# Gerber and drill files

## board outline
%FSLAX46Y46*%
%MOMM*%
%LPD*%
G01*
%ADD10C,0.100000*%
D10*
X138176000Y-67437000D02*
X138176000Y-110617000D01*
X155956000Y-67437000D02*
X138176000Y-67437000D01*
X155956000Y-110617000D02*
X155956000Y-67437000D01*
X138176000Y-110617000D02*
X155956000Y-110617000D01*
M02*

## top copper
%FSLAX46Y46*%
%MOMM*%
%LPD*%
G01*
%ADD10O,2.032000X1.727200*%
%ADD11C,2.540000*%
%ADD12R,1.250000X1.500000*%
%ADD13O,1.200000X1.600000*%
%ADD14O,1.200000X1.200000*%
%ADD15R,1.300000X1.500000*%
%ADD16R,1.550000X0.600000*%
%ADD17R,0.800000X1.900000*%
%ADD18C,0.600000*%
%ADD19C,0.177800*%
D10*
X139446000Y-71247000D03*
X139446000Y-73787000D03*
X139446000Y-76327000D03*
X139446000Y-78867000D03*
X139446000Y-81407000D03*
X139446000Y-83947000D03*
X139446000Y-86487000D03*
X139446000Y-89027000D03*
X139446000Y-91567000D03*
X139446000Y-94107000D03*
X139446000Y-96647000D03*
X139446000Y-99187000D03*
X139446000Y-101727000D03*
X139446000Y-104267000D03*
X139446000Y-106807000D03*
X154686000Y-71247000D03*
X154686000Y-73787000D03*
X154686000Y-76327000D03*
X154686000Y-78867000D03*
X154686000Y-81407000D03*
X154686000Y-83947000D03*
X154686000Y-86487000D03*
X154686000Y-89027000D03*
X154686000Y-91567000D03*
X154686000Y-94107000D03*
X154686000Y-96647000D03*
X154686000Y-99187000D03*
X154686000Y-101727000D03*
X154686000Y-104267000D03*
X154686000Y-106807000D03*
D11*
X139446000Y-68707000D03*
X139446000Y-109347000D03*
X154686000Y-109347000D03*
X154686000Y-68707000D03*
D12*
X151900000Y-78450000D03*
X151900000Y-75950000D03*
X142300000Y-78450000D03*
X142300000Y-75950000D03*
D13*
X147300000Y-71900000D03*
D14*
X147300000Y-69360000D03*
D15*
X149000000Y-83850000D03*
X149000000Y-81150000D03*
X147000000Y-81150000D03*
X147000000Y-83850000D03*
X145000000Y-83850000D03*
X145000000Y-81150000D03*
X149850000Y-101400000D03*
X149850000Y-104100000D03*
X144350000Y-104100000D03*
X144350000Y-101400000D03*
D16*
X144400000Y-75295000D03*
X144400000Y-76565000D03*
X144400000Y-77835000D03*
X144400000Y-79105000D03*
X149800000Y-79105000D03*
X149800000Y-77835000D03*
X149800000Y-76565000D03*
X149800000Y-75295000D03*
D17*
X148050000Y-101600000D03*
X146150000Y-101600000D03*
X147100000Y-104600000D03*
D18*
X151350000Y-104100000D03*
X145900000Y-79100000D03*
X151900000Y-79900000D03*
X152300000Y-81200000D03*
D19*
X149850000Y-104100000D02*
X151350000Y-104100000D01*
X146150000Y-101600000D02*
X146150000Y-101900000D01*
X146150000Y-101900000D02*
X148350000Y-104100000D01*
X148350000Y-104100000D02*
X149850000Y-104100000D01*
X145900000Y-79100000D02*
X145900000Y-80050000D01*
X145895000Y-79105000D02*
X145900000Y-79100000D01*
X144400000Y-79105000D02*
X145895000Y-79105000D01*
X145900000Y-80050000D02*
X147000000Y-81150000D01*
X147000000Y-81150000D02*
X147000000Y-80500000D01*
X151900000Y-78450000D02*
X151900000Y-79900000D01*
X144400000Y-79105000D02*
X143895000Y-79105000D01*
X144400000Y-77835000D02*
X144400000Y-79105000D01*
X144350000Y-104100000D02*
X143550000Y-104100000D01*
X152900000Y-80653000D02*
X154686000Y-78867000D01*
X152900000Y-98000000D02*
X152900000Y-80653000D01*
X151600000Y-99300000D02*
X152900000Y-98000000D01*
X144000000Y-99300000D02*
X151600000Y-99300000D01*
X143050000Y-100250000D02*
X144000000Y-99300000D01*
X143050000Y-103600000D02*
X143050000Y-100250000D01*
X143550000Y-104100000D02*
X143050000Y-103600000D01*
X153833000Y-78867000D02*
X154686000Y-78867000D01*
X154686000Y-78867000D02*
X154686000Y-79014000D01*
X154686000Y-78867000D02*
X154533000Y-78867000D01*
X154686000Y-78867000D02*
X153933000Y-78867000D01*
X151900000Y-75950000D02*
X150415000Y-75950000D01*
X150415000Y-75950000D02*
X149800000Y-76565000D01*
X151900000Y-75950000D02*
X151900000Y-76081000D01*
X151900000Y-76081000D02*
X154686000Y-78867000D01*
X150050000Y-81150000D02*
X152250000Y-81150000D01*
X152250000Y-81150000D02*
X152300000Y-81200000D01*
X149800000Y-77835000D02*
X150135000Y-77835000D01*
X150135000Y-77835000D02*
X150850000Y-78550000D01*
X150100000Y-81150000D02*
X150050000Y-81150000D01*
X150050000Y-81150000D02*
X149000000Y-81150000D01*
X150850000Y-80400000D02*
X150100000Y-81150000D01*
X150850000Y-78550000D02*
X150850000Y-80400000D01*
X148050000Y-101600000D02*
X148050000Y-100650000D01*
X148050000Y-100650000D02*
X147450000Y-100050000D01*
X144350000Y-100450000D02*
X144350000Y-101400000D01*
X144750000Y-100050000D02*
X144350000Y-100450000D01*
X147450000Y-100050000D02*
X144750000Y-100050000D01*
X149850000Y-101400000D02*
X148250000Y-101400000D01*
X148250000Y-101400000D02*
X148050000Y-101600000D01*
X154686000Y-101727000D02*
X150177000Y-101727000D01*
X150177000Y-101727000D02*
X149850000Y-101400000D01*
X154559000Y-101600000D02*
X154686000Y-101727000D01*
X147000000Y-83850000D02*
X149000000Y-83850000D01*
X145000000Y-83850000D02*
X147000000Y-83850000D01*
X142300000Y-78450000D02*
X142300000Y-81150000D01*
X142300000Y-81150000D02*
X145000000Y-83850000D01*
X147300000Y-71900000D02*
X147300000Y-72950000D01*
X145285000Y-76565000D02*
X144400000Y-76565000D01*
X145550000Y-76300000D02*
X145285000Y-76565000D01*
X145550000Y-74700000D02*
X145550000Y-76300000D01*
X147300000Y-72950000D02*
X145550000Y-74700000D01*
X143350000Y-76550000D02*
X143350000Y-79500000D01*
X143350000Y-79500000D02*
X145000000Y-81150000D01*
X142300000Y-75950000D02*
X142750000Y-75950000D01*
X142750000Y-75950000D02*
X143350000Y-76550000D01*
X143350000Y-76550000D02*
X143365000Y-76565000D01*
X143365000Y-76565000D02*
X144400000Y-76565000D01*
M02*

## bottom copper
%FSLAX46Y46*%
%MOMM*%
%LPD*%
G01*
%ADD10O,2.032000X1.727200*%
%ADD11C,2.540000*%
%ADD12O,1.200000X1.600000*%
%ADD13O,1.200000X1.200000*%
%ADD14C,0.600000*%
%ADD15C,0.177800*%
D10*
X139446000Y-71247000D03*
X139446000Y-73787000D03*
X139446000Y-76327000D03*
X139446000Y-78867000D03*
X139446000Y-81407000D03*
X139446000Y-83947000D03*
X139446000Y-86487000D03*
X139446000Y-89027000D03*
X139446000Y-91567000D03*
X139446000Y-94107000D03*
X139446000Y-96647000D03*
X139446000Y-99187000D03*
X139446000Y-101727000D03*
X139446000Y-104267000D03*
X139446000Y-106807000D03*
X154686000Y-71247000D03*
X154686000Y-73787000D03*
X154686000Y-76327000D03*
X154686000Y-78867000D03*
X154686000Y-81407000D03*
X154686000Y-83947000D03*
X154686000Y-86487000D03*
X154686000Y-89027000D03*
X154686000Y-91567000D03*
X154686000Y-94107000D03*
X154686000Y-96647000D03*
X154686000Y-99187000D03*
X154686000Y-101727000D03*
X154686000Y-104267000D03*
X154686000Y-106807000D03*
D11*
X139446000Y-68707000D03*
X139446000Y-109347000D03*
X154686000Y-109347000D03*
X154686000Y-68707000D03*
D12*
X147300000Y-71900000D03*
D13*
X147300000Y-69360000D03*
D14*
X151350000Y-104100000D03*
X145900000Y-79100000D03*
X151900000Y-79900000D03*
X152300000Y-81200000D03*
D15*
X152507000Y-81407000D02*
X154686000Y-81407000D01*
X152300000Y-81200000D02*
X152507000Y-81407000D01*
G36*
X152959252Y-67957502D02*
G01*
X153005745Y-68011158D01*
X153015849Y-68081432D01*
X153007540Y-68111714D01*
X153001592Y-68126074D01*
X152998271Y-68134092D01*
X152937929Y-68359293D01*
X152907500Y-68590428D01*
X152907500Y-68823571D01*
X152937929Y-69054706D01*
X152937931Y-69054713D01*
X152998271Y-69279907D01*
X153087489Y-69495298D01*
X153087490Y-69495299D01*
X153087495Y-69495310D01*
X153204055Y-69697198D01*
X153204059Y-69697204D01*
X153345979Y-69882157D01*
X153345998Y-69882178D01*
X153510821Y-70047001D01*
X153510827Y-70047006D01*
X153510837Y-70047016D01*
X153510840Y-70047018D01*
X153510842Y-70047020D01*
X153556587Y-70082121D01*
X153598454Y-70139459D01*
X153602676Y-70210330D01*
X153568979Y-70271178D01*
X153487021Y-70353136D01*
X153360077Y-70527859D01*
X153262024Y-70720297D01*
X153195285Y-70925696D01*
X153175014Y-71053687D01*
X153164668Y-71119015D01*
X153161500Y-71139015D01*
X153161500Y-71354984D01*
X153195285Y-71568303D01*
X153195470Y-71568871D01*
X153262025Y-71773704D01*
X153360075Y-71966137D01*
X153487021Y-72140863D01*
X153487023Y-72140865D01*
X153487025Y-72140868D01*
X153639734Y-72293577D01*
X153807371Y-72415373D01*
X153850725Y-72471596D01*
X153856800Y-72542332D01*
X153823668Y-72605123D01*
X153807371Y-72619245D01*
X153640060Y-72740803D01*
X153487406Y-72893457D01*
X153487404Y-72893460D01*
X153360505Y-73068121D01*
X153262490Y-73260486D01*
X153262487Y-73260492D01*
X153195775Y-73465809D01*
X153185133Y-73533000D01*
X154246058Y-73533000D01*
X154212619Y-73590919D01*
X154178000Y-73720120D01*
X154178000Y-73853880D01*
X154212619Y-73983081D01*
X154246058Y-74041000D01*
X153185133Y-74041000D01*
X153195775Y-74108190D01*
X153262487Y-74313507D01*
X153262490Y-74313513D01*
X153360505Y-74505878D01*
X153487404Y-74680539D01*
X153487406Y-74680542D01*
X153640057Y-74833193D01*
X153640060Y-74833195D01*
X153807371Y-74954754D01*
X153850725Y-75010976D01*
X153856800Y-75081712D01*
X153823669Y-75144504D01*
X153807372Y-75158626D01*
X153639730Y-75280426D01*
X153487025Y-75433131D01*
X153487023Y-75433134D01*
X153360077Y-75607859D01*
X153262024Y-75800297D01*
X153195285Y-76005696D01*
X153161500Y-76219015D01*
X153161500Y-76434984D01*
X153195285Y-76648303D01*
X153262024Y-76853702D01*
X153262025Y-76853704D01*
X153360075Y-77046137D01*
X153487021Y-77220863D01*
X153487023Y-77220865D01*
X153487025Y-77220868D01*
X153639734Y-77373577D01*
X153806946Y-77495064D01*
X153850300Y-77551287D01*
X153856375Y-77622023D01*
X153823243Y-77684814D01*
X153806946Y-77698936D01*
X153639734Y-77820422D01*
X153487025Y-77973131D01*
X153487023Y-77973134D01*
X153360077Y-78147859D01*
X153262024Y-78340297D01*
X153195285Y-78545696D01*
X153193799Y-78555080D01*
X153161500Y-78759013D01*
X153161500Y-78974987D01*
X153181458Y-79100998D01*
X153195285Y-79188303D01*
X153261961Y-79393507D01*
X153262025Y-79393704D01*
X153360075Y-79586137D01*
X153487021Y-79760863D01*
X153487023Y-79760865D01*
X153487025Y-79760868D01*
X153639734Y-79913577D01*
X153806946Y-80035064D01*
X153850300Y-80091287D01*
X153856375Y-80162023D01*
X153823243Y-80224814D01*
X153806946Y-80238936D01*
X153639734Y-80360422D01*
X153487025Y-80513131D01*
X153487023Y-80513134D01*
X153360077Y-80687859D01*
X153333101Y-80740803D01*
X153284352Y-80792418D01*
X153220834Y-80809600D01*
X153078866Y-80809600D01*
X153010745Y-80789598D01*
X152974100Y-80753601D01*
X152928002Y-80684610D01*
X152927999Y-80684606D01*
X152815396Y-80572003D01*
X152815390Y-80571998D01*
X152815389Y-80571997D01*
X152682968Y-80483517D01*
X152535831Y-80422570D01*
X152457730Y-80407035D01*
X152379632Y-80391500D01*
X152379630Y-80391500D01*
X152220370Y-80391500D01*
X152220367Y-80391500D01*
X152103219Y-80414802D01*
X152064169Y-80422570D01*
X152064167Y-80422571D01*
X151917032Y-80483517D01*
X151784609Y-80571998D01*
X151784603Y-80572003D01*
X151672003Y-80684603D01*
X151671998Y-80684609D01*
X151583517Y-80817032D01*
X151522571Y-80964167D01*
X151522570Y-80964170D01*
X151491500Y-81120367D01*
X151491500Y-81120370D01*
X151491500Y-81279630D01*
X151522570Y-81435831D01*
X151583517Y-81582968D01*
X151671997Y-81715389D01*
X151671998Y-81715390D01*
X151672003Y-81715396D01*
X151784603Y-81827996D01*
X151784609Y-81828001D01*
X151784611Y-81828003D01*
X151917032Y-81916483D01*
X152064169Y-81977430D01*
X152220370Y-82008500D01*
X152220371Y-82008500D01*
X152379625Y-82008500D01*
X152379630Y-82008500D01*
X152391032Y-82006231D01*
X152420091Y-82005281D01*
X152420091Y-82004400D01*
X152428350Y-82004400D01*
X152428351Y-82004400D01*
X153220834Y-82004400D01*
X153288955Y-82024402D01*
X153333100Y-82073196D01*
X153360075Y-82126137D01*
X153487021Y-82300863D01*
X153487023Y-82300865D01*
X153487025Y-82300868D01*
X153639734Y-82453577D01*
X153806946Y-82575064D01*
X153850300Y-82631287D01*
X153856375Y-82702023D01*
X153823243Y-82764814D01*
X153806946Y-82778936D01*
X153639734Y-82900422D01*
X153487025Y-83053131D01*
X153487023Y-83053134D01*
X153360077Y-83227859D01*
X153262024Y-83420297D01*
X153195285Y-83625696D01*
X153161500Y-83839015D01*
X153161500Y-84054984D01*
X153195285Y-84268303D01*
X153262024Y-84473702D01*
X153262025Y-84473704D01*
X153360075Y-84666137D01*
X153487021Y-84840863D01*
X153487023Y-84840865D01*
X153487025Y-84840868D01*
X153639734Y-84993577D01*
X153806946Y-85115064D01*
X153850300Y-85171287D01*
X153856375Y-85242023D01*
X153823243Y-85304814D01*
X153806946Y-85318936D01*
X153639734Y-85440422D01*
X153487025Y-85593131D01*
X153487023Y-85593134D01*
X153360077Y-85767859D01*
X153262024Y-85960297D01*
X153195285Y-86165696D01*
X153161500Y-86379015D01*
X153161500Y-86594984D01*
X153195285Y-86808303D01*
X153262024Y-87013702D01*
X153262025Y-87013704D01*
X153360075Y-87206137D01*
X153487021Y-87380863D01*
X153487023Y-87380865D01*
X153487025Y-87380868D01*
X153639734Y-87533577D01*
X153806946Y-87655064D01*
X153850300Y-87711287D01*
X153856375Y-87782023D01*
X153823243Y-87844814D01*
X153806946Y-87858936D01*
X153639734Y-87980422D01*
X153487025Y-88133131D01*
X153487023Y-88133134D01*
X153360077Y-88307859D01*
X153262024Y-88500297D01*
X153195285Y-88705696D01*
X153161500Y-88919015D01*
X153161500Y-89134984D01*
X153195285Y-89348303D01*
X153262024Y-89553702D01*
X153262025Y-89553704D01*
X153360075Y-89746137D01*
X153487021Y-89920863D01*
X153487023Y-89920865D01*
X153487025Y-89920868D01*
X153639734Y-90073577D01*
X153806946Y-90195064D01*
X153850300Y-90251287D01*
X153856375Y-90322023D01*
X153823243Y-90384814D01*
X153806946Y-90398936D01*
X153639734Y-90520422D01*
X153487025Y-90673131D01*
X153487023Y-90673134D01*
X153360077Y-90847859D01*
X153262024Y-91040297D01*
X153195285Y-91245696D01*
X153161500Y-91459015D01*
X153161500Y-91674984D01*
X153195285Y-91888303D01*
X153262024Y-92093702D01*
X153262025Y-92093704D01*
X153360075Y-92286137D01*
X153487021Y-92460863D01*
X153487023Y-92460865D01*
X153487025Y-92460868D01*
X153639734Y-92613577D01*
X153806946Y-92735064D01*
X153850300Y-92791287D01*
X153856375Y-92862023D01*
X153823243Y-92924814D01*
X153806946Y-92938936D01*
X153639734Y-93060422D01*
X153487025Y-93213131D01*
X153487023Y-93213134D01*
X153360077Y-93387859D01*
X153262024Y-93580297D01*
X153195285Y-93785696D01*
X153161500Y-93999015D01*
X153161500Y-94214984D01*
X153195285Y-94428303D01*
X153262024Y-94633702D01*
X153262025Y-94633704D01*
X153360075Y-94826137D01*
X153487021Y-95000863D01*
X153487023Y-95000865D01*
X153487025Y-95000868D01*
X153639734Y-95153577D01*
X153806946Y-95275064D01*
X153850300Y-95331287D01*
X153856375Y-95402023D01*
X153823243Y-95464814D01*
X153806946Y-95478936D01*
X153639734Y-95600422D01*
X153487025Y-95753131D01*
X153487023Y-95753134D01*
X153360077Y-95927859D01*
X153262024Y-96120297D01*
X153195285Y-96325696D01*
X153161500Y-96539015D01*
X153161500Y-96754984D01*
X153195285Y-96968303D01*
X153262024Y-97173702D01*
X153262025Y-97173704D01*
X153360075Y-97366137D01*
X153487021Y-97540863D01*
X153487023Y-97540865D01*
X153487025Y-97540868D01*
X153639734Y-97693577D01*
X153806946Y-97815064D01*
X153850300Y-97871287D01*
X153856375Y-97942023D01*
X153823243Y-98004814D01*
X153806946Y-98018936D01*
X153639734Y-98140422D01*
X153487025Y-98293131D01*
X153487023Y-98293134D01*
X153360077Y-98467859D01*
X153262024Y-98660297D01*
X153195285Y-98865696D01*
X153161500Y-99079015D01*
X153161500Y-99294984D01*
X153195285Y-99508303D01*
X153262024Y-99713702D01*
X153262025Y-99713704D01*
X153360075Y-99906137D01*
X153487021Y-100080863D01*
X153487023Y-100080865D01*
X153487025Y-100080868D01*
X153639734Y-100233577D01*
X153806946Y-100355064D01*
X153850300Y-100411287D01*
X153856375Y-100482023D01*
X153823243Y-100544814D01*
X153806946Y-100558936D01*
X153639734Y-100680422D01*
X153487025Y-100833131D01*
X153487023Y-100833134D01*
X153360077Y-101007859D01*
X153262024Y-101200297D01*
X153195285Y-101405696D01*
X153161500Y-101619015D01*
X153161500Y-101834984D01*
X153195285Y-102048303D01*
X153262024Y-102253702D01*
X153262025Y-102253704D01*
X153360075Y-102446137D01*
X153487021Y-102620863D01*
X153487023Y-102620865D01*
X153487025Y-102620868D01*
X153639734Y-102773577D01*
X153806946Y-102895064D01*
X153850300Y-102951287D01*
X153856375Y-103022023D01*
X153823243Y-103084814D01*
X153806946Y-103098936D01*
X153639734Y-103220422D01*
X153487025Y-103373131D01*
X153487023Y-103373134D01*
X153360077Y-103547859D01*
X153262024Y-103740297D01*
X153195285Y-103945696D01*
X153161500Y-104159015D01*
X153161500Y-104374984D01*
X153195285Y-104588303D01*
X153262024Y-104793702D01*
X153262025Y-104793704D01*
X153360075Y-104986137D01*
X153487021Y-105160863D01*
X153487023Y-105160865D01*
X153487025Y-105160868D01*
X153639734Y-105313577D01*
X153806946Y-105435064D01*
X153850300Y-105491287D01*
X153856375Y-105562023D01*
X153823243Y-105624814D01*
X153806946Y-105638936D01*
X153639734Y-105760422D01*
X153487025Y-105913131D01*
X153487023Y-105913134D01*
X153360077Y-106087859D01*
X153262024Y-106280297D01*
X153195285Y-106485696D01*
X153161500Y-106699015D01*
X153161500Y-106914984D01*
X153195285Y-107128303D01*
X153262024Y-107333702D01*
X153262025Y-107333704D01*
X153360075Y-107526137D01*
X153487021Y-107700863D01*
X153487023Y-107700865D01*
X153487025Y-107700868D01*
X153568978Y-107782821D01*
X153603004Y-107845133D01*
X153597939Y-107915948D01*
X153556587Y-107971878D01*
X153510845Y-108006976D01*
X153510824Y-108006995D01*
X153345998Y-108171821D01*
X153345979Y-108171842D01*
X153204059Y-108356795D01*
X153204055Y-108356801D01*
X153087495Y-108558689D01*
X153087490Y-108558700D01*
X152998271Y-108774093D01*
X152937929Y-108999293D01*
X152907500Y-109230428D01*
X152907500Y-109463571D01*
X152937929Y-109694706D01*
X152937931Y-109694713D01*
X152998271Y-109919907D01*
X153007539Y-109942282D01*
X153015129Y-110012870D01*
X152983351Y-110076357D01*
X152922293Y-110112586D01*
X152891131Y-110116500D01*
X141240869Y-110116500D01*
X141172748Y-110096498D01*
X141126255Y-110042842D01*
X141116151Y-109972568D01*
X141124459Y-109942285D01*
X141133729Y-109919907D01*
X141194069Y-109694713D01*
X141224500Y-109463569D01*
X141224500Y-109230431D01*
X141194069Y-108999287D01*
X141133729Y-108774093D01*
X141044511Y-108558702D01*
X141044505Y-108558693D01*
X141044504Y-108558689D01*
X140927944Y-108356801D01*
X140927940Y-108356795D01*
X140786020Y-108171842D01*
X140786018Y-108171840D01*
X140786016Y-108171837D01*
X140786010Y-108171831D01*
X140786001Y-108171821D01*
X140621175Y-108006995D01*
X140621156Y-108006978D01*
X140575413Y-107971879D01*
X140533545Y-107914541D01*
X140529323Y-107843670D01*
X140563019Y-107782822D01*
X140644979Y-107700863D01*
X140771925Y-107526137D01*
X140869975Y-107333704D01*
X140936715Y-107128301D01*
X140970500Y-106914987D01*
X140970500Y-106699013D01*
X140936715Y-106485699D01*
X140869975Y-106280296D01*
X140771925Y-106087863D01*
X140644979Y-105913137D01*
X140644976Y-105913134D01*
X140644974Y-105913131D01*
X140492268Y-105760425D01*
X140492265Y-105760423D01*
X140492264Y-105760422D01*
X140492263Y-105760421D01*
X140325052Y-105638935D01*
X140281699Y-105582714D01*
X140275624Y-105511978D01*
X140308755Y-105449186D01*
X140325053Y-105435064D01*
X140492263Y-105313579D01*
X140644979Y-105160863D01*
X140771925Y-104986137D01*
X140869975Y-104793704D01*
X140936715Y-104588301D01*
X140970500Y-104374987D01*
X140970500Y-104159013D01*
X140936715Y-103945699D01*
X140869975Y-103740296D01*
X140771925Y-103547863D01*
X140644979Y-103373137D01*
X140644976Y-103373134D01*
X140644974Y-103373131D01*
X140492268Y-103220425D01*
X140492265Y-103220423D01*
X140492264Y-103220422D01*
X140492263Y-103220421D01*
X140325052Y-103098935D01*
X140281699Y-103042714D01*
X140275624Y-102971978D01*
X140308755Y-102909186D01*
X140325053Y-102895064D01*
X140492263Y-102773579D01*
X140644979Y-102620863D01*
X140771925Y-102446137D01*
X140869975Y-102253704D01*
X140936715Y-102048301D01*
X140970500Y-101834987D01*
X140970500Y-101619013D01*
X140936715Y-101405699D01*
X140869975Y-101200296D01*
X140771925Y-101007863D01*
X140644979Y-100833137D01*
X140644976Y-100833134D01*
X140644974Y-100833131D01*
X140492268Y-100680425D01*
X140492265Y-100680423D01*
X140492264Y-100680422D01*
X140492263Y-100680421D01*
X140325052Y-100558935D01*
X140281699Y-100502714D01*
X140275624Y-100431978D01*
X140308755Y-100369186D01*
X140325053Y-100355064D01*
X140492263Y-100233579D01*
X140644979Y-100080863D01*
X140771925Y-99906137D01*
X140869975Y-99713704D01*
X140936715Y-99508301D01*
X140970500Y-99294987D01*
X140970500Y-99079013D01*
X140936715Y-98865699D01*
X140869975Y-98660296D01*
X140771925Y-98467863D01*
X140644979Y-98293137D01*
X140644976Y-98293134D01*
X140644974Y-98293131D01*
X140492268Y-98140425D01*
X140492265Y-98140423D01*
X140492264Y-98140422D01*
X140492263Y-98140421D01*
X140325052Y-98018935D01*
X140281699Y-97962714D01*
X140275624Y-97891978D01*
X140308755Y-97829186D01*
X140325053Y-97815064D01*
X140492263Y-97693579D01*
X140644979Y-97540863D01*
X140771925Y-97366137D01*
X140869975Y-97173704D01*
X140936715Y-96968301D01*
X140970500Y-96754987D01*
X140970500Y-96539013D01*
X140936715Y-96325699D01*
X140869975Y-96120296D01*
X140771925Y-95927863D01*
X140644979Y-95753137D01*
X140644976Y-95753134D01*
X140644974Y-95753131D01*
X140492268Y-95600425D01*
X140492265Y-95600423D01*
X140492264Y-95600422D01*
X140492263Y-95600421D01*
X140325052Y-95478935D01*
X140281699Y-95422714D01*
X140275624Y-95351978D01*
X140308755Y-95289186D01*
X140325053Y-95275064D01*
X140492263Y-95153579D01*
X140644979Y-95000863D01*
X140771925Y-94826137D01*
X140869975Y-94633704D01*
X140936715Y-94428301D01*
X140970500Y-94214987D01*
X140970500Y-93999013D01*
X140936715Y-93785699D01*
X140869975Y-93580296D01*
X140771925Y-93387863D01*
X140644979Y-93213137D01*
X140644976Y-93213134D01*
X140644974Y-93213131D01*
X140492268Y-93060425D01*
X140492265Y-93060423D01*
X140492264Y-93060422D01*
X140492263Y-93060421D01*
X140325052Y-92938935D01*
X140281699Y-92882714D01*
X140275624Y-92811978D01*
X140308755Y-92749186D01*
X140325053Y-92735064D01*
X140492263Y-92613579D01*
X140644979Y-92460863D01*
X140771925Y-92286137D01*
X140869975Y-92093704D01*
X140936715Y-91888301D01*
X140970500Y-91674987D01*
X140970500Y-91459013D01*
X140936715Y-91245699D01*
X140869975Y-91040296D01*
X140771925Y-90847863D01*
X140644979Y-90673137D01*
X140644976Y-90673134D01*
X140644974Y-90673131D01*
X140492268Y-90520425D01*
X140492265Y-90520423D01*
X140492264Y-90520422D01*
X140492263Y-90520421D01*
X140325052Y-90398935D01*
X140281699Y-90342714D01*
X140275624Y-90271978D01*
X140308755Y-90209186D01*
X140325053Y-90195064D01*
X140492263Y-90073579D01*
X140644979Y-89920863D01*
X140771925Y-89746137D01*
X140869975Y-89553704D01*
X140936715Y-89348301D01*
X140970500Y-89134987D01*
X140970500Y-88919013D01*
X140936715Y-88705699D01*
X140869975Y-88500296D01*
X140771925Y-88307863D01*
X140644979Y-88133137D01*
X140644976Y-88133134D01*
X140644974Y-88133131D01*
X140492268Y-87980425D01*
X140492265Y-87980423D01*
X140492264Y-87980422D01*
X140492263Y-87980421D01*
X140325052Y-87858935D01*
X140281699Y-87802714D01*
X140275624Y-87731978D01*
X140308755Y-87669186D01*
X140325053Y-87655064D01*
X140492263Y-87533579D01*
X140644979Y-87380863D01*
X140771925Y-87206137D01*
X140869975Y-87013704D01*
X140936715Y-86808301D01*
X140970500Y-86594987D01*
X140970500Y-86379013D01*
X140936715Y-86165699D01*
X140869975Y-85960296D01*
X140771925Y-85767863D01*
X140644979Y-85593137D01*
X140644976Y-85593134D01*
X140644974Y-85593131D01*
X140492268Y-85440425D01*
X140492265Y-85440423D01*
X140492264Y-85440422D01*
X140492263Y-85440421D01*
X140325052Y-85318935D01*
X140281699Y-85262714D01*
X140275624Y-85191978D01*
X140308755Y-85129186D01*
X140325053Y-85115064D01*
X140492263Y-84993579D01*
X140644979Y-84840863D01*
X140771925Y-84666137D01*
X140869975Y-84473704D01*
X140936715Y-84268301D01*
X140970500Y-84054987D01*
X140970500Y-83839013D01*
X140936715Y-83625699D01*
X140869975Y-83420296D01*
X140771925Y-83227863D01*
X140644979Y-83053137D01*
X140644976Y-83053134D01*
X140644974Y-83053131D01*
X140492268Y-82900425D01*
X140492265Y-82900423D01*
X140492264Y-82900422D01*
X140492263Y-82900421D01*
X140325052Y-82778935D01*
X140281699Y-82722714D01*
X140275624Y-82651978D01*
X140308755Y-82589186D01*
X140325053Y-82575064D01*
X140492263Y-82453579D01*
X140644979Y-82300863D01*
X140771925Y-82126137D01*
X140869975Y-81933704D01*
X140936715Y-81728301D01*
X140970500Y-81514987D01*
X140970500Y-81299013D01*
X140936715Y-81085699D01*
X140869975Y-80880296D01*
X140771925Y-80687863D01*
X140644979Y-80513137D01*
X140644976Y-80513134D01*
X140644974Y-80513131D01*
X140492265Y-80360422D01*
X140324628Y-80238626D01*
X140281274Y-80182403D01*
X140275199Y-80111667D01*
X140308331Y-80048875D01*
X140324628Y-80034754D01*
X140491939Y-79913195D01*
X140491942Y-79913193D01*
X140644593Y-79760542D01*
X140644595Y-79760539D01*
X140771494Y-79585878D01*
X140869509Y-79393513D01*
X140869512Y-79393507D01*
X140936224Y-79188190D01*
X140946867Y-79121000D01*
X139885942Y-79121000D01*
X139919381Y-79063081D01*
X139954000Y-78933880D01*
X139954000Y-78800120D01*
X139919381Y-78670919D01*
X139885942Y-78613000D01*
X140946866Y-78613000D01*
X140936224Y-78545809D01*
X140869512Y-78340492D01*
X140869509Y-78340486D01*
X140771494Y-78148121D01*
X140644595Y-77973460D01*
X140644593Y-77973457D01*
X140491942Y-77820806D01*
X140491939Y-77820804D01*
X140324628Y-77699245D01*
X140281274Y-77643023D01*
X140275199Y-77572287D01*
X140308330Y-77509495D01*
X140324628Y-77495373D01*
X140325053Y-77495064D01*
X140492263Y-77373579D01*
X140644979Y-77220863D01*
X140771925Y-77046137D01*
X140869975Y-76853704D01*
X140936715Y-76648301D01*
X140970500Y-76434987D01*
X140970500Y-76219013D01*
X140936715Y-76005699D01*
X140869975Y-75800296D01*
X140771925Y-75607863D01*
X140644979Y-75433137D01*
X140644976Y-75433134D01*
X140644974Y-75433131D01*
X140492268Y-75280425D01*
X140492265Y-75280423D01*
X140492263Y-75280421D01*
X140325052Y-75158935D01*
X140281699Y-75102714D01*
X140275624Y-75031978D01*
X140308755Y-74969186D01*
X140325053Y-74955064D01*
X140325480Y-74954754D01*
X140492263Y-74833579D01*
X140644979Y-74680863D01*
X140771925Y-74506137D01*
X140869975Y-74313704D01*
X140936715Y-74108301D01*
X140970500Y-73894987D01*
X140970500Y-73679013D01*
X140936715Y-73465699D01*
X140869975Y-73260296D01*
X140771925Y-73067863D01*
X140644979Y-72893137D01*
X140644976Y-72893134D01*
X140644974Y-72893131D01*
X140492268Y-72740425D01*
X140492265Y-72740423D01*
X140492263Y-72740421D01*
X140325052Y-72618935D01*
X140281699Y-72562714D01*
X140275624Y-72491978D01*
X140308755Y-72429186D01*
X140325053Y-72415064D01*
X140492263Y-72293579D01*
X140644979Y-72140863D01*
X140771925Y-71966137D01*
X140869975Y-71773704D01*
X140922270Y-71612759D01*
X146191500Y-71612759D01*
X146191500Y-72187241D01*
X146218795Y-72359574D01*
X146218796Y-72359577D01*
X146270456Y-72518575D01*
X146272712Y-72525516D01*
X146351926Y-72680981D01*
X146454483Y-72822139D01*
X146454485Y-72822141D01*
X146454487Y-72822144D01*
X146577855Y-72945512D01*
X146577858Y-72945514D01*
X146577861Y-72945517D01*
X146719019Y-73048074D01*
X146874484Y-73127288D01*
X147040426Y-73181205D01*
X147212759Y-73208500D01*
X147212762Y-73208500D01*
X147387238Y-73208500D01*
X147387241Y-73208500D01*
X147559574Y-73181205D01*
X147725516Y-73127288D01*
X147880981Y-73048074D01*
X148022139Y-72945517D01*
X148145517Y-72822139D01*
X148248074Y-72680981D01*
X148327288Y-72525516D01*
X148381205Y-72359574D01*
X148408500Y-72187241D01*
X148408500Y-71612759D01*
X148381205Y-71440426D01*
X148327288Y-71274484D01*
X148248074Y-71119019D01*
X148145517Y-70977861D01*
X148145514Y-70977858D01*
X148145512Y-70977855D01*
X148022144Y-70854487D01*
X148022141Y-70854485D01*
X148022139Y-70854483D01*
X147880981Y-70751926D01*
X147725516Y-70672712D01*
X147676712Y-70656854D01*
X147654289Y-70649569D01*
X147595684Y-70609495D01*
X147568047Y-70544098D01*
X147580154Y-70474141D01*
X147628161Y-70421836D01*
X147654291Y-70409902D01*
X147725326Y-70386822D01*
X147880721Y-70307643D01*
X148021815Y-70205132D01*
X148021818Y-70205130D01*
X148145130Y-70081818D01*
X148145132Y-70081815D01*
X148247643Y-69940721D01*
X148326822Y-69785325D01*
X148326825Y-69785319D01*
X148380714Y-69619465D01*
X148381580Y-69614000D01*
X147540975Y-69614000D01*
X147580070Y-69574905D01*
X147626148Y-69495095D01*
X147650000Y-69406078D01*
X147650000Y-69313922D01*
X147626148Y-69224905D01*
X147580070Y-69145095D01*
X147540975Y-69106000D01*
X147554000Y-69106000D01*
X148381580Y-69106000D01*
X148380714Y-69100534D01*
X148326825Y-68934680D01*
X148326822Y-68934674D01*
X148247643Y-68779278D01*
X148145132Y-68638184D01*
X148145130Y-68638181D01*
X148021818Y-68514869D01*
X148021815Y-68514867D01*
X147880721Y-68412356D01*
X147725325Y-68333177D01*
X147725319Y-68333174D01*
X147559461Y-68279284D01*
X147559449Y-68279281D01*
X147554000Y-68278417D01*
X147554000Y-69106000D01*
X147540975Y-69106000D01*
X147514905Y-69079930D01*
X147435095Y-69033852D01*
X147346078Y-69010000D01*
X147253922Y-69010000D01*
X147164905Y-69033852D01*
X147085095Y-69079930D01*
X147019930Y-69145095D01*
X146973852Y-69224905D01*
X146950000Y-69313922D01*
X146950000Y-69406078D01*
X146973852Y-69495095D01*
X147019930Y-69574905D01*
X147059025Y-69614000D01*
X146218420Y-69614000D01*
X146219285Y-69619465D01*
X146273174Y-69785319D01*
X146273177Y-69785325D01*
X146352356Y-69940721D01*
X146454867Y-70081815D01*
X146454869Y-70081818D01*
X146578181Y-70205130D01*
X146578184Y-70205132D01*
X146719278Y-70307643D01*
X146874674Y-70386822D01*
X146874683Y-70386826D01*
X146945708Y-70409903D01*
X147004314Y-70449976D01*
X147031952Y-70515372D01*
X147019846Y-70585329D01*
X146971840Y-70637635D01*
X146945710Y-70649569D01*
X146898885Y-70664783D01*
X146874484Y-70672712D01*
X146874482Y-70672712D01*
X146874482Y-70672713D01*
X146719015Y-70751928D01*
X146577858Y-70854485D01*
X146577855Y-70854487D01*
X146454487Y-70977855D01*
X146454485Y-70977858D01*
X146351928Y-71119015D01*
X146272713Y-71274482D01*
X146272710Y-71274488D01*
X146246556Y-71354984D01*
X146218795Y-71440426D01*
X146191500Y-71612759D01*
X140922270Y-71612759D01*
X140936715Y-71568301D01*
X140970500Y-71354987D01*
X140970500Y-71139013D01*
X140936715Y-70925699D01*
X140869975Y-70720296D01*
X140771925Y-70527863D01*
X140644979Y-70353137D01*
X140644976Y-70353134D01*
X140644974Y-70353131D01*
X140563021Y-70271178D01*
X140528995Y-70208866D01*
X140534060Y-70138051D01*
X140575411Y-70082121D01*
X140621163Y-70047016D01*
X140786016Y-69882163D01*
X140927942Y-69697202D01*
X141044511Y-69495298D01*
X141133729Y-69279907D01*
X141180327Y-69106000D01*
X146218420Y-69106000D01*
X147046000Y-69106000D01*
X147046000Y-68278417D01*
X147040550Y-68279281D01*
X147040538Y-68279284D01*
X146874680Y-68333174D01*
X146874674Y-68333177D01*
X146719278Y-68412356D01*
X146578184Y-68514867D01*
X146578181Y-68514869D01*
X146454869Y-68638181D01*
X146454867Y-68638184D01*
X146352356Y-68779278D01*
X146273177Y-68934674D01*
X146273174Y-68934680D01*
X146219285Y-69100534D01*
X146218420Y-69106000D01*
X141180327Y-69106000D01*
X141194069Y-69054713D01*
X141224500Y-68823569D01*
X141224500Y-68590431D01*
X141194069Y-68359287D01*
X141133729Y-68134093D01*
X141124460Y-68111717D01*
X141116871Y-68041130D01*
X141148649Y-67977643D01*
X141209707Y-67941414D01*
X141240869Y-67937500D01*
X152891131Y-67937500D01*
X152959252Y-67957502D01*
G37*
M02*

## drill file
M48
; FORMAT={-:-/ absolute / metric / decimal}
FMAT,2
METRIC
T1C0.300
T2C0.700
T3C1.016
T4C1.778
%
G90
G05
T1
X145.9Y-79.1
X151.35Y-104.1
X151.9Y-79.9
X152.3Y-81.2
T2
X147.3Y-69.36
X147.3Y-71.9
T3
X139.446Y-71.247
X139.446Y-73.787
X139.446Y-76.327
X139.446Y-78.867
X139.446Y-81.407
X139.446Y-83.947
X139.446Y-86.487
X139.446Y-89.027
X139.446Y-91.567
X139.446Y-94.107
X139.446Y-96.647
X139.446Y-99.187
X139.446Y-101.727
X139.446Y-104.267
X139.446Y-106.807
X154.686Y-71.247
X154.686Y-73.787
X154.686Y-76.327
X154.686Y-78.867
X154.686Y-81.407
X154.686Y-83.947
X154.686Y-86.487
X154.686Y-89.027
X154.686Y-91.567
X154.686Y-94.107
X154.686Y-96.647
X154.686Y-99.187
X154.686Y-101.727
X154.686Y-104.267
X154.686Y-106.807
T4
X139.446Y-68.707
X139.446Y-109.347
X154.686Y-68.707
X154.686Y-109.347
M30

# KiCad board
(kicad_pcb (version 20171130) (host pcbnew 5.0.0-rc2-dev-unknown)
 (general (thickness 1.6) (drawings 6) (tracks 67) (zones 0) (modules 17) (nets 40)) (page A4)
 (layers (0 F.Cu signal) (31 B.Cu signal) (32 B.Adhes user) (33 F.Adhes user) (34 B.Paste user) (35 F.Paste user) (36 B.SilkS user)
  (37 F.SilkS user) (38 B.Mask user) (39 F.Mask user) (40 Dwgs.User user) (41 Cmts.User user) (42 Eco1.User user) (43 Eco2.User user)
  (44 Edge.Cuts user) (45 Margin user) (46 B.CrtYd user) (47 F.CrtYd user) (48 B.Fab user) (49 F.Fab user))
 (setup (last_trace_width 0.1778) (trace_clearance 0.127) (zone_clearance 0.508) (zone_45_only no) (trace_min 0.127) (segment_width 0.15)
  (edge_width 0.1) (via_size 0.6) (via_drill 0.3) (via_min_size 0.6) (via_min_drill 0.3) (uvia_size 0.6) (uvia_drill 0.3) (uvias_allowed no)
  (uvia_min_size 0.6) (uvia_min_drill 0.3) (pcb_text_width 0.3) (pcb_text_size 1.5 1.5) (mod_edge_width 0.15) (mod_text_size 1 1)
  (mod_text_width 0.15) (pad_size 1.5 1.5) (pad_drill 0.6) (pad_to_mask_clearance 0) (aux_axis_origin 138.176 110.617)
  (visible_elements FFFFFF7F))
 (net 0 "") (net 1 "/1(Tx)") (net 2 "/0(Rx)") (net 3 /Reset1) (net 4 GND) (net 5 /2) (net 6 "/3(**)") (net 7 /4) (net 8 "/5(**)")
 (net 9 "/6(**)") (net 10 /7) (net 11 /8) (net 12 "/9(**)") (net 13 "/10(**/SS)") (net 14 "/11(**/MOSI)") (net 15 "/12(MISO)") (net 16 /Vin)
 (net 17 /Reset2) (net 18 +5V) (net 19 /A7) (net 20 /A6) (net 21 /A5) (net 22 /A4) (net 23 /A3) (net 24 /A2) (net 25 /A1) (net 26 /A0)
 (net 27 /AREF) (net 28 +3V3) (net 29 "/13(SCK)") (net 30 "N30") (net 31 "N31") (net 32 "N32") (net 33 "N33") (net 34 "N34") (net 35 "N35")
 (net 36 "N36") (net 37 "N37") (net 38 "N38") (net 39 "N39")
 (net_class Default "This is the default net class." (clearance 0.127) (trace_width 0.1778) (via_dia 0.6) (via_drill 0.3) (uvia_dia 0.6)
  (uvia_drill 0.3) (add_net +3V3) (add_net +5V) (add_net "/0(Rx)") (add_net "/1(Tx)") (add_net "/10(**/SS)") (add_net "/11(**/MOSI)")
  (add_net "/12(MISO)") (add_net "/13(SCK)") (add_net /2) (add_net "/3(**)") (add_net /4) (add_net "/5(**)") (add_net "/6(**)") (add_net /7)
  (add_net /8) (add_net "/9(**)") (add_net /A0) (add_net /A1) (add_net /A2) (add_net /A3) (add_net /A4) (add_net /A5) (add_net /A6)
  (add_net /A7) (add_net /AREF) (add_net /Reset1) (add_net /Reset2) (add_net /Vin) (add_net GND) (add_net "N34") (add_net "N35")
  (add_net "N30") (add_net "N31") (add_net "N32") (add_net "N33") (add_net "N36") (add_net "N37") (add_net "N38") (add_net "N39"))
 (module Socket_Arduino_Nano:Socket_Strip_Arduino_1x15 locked (layer F.Cu) (at 139.446 71.247 270)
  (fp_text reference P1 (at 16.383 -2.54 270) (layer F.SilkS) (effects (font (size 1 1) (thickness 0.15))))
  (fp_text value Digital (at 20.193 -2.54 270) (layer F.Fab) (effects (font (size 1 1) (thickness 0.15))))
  (pad 1 thru_hole oval (at 0 0 270) (size 1.7272 2.032) (drill 1.016) (layers *.Cu *.Mask F.SilkS) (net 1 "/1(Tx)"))
  (pad 2 thru_hole oval (at 2.54 0 270) (size 1.7272 2.032) (drill 1.016) (layers *.Cu *.Mask F.SilkS) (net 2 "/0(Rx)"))
  (pad 3 thru_hole oval (at 5.08 0 270) (size 1.7272 2.032) (drill 1.016) (layers *.Cu *.Mask F.SilkS) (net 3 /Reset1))
  (pad 4 thru_hole oval (at 7.62 0 270) (size 1.7272 2.032) (drill 1.016) (layers *.Cu *.Mask F.SilkS) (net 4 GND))
  (pad 5 thru_hole oval (at 10.16 0 270) (size 1.7272 2.032) (drill 1.016) (layers *.Cu *.Mask F.SilkS) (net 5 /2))
  (pad 6 thru_hole oval (at 12.7 0 270) (size 1.7272 2.032) (drill 1.016) (layers *.Cu *.Mask F.SilkS) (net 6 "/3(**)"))
  (pad 7 thru_hole oval (at 15.24 0 270) (size 1.7272 2.032) (drill 1.016) (layers *.Cu *.Mask F.SilkS) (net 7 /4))
  (pad 8 thru_hole oval (at 17.78 0 270) (size 1.7272 2.032) (drill 1.016) (layers *.Cu *.Mask F.SilkS) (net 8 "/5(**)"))
  (pad 9 thru_hole oval (at 20.32 0 270) (size 1.7272 2.032) (drill 1.016) (layers *.Cu *.Mask F.SilkS) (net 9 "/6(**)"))
  (pad 10 thru_hole oval (at 22.86 0 270) (size 1.7272 2.032) (drill 1.016) (layers *.Cu *.Mask F.SilkS) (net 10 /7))
  (pad 11 thru_hole oval (at 25.4 0 270) (size 1.7272 2.032) (drill 1.016) (layers *.Cu *.Mask F.SilkS) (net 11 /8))
  (pad 12 thru_hole oval (at 27.94 0 270) (size 1.7272 2.032) (drill 1.016) (layers *.Cu *.Mask F.SilkS) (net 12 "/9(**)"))
  (pad 13 thru_hole oval (at 30.48 0 270) (size 1.7272 2.032) (drill 1.016) (layers *.Cu *.Mask F.SilkS) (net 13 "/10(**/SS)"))
  (pad 14 thru_hole oval (at 33.02 0 270) (size 1.7272 2.032) (drill 1.016) (layers *.Cu *.Mask F.SilkS) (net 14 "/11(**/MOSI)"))
  (pad 15 thru_hole oval (at 35.56 0 270) (size 1.7272 2.032) (drill 1.016) (layers *.Cu *.Mask F.SilkS) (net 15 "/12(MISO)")))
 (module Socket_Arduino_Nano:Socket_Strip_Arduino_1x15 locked (layer F.Cu) (at 154.686 71.247 270)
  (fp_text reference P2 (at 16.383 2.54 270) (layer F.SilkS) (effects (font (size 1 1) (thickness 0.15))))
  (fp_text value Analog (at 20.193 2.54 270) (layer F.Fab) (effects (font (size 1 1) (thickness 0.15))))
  (pad 1 thru_hole oval (at 0 0 270) (size 1.7272 2.032) (drill 1.016) (layers *.Cu *.Mask F.SilkS) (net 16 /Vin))
  (pad 2 thru_hole oval (at 2.54 0 270) (size 1.7272 2.032) (drill 1.016) (layers *.Cu *.Mask F.SilkS) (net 4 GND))
  (pad 3 thru_hole oval (at 5.08 0 270) (size 1.7272 2.032) (drill 1.016) (layers *.Cu *.Mask F.SilkS) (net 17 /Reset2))
  (pad 4 thru_hole oval (at 7.62 0 270) (size 1.7272 2.032) (drill 1.016) (layers *.Cu *.Mask F.SilkS) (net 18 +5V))
  (pad 5 thru_hole oval (at 10.16 0 270) (size 1.7272 2.032) (drill 1.016) (layers *.Cu *.Mask F.SilkS) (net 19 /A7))
  (pad 6 thru_hole oval (at 12.7 0 270) (size 1.7272 2.032) (drill 1.016) (layers *.Cu *.Mask F.SilkS) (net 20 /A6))
  (pad 7 thru_hole oval (at 15.24 0 270) (size 1.7272 2.032) (drill 1.016) (layers *.Cu *.Mask F.SilkS) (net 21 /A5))
  (pad 8 thru_hole oval (at 17.78 0 270) (size 1.7272 2.032) (drill 1.016) (layers *.Cu *.Mask F.SilkS) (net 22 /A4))
  (pad 9 thru_hole oval (at 20.32 0 270) (size 1.7272 2.032) (drill 1.016) (layers *.Cu *.Mask F.SilkS) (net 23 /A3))
  (pad 10 thru_hole oval (at 22.86 0 270) (size 1.7272 2.032) (drill 1.016) (layers *.Cu *.Mask F.SilkS) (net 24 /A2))
  (pad 11 thru_hole oval (at 25.4 0 270) (size 1.7272 2.032) (drill 1.016) (layers *.Cu *.Mask F.SilkS) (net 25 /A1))
  (pad 12 thru_hole oval (at 27.94 0 270) (size 1.7272 2.032) (drill 1.016) (layers *.Cu *.Mask F.SilkS) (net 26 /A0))
  (pad 13 thru_hole oval (at 30.48 0 270) (size 1.7272 2.032) (drill 1.016) (layers *.Cu *.Mask F.SilkS) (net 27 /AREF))
  (pad 14 thru_hole oval (at 33.02 0 270) (size 1.7272 2.032) (drill 1.016) (layers *.Cu *.Mask F.SilkS) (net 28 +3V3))
  (pad 15 thru_hole oval (at 35.56 0 270) (size 1.7272 2.032) (drill 1.016) (layers *.Cu *.Mask F.SilkS) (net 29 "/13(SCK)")))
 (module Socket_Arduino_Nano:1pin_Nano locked (layer F.Cu) (at 139.446 68.707)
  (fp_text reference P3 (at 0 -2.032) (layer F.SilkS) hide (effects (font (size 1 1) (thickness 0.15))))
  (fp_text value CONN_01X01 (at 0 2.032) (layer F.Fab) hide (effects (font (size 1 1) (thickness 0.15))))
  (pad 1 thru_hole circle (at 0 0) (size 2.54 2.54) (drill 1.778) (layers *.Cu *.Mask F.SilkS) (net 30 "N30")))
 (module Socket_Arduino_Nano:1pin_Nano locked (layer F.Cu) (at 139.446 109.347)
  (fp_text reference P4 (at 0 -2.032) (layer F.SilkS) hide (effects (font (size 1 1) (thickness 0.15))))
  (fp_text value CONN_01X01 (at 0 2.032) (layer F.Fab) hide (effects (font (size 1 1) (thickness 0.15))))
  (pad 1 thru_hole circle (at 0 0) (size 2.54 2.54) (drill 1.778) (layers *.Cu *.Mask F.SilkS) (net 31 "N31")))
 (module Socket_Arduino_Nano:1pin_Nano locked (layer F.Cu) (at 154.686 109.347)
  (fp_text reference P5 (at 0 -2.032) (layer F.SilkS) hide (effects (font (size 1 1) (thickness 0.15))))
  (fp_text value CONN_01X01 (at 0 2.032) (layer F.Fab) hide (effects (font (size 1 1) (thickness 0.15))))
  (pad 1 thru_hole circle (at 0 0) (size 2.54 2.54) (drill 1.778) (layers *.Cu *.Mask F.SilkS) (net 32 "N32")))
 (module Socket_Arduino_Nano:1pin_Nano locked (layer F.Cu) (at 154.686 68.707)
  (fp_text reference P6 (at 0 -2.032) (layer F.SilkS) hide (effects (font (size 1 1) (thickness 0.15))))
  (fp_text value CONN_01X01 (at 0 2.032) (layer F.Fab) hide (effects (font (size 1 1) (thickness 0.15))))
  (pad 1 thru_hole circle (at 0 0) (size 2.54 2.54) (drill 1.778) (layers *.Cu *.Mask F.SilkS) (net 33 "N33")))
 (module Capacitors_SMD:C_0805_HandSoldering (layer F.Cu) (at 151.9 77.2 90)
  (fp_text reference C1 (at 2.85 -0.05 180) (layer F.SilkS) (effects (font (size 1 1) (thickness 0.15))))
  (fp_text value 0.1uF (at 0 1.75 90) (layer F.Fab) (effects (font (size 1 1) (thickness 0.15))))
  (pad 1 smd rect (at -1.25 0 90) (size 1.5 1.25) (layers F.Cu F.Paste F.Mask) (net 4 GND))
  (pad 2 smd rect (at 1.25 0 90) (size 1.5 1.25) (layers F.Cu F.Paste F.Mask) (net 18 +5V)))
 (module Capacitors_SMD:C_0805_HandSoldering (layer F.Cu) (at 142.3 77.2 90)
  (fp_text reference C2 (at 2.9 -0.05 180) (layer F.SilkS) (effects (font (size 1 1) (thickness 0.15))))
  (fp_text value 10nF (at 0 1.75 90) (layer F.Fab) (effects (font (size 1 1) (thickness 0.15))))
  (pad 1 smd rect (at -1.25 0 90) (size 1.5 1.25) (layers F.Cu F.Paste F.Mask) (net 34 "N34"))
  (pad 2 smd rect (at 1.25 0 90) (size 1.5 1.25) (layers F.Cu F.Paste F.Mask) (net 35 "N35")))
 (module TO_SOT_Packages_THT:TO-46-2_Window (layer F.Cu) (at 147.3 71.9 90)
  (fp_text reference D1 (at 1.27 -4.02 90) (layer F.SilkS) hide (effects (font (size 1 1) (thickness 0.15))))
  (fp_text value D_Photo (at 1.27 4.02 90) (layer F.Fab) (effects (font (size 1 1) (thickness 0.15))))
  (pad 1 thru_hole oval (at 0 0 90) (size 1.6 1.2) (drill 0.7) (layers *.Cu *.Mask) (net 35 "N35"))
  (pad 2 thru_hole oval (at 2.54 0 90) (size 1.2 1.2) (drill 0.7) (layers *.Cu *.Mask) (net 4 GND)))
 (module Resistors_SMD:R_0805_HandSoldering (layer F.Cu) (at 149 82.5 90)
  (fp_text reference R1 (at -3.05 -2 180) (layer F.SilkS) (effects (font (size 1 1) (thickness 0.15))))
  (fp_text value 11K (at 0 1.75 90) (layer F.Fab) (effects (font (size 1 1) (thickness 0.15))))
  (pad 1 smd rect (at -1.35 0 90) (size 1.5 1.3) (layers F.Cu F.Paste F.Mask) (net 34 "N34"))
  (pad 2 smd rect (at 1.35 0 90) (size 1.5 1.3) (layers F.Cu F.Paste F.Mask) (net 19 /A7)))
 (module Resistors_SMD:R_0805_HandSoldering (layer F.Cu) (at 147 82.5 270)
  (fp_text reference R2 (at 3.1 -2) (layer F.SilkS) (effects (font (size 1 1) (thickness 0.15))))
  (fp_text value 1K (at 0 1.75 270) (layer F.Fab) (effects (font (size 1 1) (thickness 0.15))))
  (pad 1 smd rect (at -1.35 0 270) (size 1.5 1.3) (layers F.Cu F.Paste F.Mask) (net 4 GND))
  (pad 2 smd rect (at 1.35 0 270) (size 1.5 1.3) (layers F.Cu F.Paste F.Mask) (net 34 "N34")))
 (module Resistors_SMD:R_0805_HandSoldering (layer F.Cu) (at 145 82.5 90)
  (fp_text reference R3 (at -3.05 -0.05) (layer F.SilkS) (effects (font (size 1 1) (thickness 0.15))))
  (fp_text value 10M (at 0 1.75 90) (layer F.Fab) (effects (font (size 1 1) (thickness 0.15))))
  (pad 1 smd rect (at -1.35 0 90) (size 1.5 1.3) (layers F.Cu F.Paste F.Mask) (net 34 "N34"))
  (pad 2 smd rect (at 1.35 0 90) (size 1.5 1.3) (layers F.Cu F.Paste F.Mask) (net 35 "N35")))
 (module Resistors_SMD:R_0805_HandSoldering (layer F.Cu) (at 149.85 102.75 270)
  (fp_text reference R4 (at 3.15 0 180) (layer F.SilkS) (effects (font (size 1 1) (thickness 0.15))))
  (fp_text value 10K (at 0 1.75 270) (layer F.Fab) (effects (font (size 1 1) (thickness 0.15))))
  (pad 1 smd rect (at -1.35 0 270) (size 1.5 1.3) (layers F.Cu F.Paste F.Mask) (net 27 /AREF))
  (pad 2 smd rect (at 1.35 0 270) (size 1.5 1.3) (layers F.Cu F.Paste F.Mask) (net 4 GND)))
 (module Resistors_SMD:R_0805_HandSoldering (layer F.Cu) (at 144.35 102.75 90)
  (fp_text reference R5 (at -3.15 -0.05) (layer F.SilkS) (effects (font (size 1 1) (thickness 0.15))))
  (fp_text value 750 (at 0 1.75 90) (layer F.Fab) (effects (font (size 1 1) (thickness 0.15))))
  (pad 1 smd rect (at -1.35 0 90) (size 1.5 1.3) (layers F.Cu F.Paste F.Mask) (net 18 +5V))
  (pad 2 smd rect (at 1.35 0 90) (size 1.5 1.3) (layers F.Cu F.Paste F.Mask) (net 27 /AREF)))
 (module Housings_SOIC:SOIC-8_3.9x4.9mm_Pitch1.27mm (layer F.Cu) (at 147.1 77.2)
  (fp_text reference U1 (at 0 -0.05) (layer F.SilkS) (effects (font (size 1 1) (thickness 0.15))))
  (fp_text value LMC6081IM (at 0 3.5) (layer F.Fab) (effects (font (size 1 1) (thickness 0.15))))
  (pad 1 smd rect (at -2.7 -1.905) (size 1.55 0.6) (layers F.Cu F.Paste F.Mask) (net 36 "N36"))
  (pad 2 smd rect (at -2.7 -0.635) (size 1.55 0.6) (layers F.Cu F.Paste F.Mask) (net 35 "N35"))
  (pad 3 smd rect (at -2.7 0.635) (size 1.55 0.6) (layers F.Cu F.Paste F.Mask) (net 4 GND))
  (pad 4 smd rect (at -2.7 1.905) (size 1.55 0.6) (layers F.Cu F.Paste F.Mask) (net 4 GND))
  (pad 5 smd rect (at 2.7 1.905) (size 1.55 0.6) (layers F.Cu F.Paste F.Mask) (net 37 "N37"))
  (pad 6 smd rect (at 2.7 0.635) (size 1.55 0.6) (layers F.Cu F.Paste F.Mask) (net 19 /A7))
  (pad 7 smd rect (at 2.7 -0.635) (size 1.55 0.6) (layers F.Cu F.Paste F.Mask) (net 18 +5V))
  (pad 8 smd rect (at 2.7 -1.905) (size 1.55 0.6) (layers F.Cu F.Paste F.Mask) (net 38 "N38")))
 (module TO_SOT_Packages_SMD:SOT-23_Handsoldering (layer F.Cu) (at 147.1 103.1 270)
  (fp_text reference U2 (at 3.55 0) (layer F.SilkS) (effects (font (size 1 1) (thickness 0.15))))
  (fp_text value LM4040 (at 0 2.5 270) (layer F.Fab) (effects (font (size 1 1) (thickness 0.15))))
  (pad 1 smd rect (at -1.5 -0.95 270) (size 1.9 0.8) (layers F.Cu F.Paste F.Mask) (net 27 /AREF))
  (pad 2 smd rect (at -1.5 0.95 270) (size 1.9 0.8) (layers F.Cu F.Paste F.Mask) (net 4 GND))
  (pad 3 smd rect (at 1.5 0 270) (size 1.9 0.8) (layers F.Cu F.Paste F.Mask) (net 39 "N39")))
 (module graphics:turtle (layer F.Cu) (at 147 93)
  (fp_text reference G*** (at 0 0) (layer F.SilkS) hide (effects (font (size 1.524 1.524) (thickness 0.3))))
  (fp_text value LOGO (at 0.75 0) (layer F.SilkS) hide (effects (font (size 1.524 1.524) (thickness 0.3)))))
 (gr_line (start 138.176 67.437) (end 138.176 110.617) (angle 90) (layer Edge.Cuts) (width 0.1))
 (gr_line (start 155.956 67.437) (end 138.176 67.437) (angle 90) (layer Edge.Cuts) (width 0.1))
 (gr_line (start 155.956 110.617) (end 155.956 67.437) (angle 90) (layer Edge.Cuts) (width 0.1))
 (gr_line (start 138.176 110.617) (end 155.956 110.617) (angle 90) (layer Edge.Cuts) (width 0.1))
 (segment (start 149.85 104.1) (end 151.35 104.1) (width 0.1778) (layer F.Cu) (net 4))
 (via (at 151.35 104.1) (size 0.6) (drill 0.3) (layers F.Cu B.Cu) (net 4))
 (segment (start 146.15 101.6) (end 146.15 101.9) (width 0.1778) (layer F.Cu) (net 4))
 (segment (start 146.15 101.9) (end 148.35 104.1) (width 0.1778) (layer F.Cu) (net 4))
 (segment (start 148.35 104.1) (end 149.85 104.1) (width 0.1778) (layer F.Cu) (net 4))
 (segment (start 145.9 79.1) (end 145.9 80.05) (width 0.1778) (layer F.Cu) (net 4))
 (segment (start 145.895 79.105) (end 145.9 79.1) (width 0.1778) (layer F.Cu) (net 4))
 (via (at 145.9 79.1) (size 0.6) (drill 0.3) (layers F.Cu B.Cu) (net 4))
 (segment (start 144.4 79.105) (end 145.895 79.105) (width 0.1778) (layer F.Cu) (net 4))
 (segment (start 145.9 80.05) (end 147 81.15) (width 0.1778) (layer F.Cu) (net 4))
 (segment (start 147 81.15) (end 147 80.5) (width 0.1778) (layer F.Cu) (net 4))
 (segment (start 151.9 78.45) (end 151.9 79.9) (width 0.1778) (layer F.Cu) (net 4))
 (via (at 151.9 79.9) (size 0.6) (drill 0.3) (layers F.Cu B.Cu) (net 4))
 (segment (start 144.4 79.105) (end 143.895 79.105) (width 0.1778) (layer F.Cu) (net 4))
 (segment (start 144.4 77.835) (end 144.4 79.105) (width 0.1778) (layer F.Cu) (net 4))
 (segment (start 144.35 104.1) (end 143.55 104.1) (width 0.1778) (layer F.Cu) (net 18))
 (segment (start 152.9 80.653) (end 154.686 78.867) (width 0.1778) (layer F.Cu) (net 18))
 (segment (start 152.9 98) (end 152.9 80.653) (width 0.1778) (layer F.Cu) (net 18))
 (segment (start 151.6 99.3) (end 152.9 98) (width 0.1778) (layer F.Cu) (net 18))
 (segment (start 144 99.3) (end 151.6 99.3) (width 0.1778) (layer F.Cu) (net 18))
 (segment (start 143.05 100.25) (end 144 99.3) (width 0.1778) (layer F.Cu) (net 18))
 (segment (start 143.05 103.6) (end 143.05 100.25) (width 0.1778) (layer F.Cu) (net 18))
 (segment (start 143.55 104.1) (end 143.05 103.6) (width 0.1778) (layer F.Cu) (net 18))
 (segment (start 153.833 78.867) (end 154.686 78.867) (width 0.1778) (layer F.Cu) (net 18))
 (segment (start 154.686 78.867) (end 154.686 79.014) (width 0.1778) (layer F.Cu) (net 18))
 (segment (start 154.686 78.867) (end 154.533 78.867) (width 0.1778) (layer F.Cu) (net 18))
 (segment (start 154.686 78.867) (end 153.933 78.867) (width 0.1778) (layer F.Cu) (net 18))
 (segment (start 151.9 75.95) (end 150.415 75.95) (width 0.1778) (layer F.Cu) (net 18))
 (segment (start 150.415 75.95) (end 149.8 76.565) (width 0.1778) (layer F.Cu) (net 18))
 (segment (start 151.9 75.95) (end 151.9 76.081) (width 0.1778) (layer F.Cu) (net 18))
 (segment (start 151.9 76.081) (end 154.686 78.867) (width 0.1778) (layer F.Cu) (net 18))
 (segment (start 150.05 81.15) (end 152.25 81.15) (width 0.1778) (layer F.Cu) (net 19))
 (segment (start 152.507 81.407) (end 154.686 81.407) (width 0.1778) (layer B.Cu) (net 19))
 (segment (start 152.3 81.2) (end 152.507 81.407) (width 0.1778) (layer B.Cu) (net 19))
 (via (at 152.3 81.2) (size 0.6) (drill 0.3) (layers F.Cu B.Cu) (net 19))
 (segment (start 152.25 81.15) (end 152.3 81.2) (width 0.1778) (layer F.Cu) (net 19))
 (segment (start 149.8 77.835) (end 150.135 77.835) (width 0.1778) (layer F.Cu) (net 19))
 (segment (start 150.135 77.835) (end 150.85 78.55) (width 0.1778) (layer F.Cu) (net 19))
 (segment (start 150.1 81.15) (end 150.05 81.15) (width 0.1778) (layer F.Cu) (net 19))
 (segment (start 150.05 81.15) (end 149 81.15) (width 0.1778) (layer F.Cu) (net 19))
 (segment (start 150.85 80.4) (end 150.1 81.15) (width 0.1778) (layer F.Cu) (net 19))
 (segment (start 150.85 78.55) (end 150.85 80.4) (width 0.1778) (layer F.Cu) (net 19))
 (segment (start 148.05 101.6) (end 148.05 100.65) (width 0.1778) (layer F.Cu) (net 27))
 (segment (start 148.05 100.65) (end 147.45 100.05) (width 0.1778) (layer F.Cu) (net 27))
 (segment (start 144.35 100.45) (end 144.35 101.4) (width 0.1778) (layer F.Cu) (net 27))
 (segment (start 144.75 100.05) (end 144.35 100.45) (width 0.1778) (layer F.Cu) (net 27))
 (segment (start 147.45 100.05) (end 144.75 100.05) (width 0.1778) (layer F.Cu) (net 27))
 (segment (start 149.85 101.4) (end 148.25 101.4) (width 0.1778) (layer F.Cu) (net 27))
 (segment (start 148.25 101.4) (end 148.05 101.6) (width 0.1778) (layer F.Cu) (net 27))
 (segment (start 154.686 101.727) (end 150.177 101.727) (width 0.1778) (layer F.Cu) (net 27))
 (segment (start 150.177 101.727) (end 149.85 101.4) (width 0.1778) (layer F.Cu) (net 27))
 (segment (start 154.559 101.6) (end 154.686 101.727) (width 0.1778) (layer F.Cu) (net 27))
 (segment (start 147 83.85) (end 149 83.85) (width 0.1778) (layer F.Cu) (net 34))
 (segment (start 145 83.85) (end 147 83.85) (width 0.1778) (layer F.Cu) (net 34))
 (segment (start 142.3 78.45) (end 142.3 81.15) (width 0.1778) (layer F.Cu) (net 34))
 (segment (start 142.3 81.15) (end 145 83.85) (width 0.1778) (layer F.Cu) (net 34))
 (segment (start 147.3 71.9) (end 147.3 72.95) (width 0.1778) (layer F.Cu) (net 35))
 (segment (start 145.285 76.565) (end 144.4 76.565) (width 0.1778) (layer F.Cu) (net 35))
 (segment (start 145.55 76.3) (end 145.285 76.565) (width 0.1778) (layer F.Cu) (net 35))
 (segment (start 145.55 74.7) (end 145.55 76.3) (width 0.1778) (layer F.Cu) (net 35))
 (segment (start 147.3 72.95) (end 145.55 74.7) (width 0.1778) (layer F.Cu) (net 35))
 (segment (start 143.35 76.55) (end 143.35 79.5) (width 0.1778) (layer F.Cu) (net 35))
 (segment (start 143.35 79.5) (end 145 81.15) (width 0.1778) (layer F.Cu) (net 35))
 (segment (start 142.3 75.95) (end 142.75 75.95) (width 0.1778) (layer F.Cu) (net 35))
 (segment (start 142.75 75.95) (end 143.35 76.55) (width 0.1778) (layer F.Cu) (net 35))
 (segment (start 143.35 76.55) (end 143.365 76.565) (width 0.1778) (layer F.Cu) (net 35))
 (segment (start 143.365 76.565) (end 144.4 76.565) (width 0.1778) (layer F.Cu) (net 35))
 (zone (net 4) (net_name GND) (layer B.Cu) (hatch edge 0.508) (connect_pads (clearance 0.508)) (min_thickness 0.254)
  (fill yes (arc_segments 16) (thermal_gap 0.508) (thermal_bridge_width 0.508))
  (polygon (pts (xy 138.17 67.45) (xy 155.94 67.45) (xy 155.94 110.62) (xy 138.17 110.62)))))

